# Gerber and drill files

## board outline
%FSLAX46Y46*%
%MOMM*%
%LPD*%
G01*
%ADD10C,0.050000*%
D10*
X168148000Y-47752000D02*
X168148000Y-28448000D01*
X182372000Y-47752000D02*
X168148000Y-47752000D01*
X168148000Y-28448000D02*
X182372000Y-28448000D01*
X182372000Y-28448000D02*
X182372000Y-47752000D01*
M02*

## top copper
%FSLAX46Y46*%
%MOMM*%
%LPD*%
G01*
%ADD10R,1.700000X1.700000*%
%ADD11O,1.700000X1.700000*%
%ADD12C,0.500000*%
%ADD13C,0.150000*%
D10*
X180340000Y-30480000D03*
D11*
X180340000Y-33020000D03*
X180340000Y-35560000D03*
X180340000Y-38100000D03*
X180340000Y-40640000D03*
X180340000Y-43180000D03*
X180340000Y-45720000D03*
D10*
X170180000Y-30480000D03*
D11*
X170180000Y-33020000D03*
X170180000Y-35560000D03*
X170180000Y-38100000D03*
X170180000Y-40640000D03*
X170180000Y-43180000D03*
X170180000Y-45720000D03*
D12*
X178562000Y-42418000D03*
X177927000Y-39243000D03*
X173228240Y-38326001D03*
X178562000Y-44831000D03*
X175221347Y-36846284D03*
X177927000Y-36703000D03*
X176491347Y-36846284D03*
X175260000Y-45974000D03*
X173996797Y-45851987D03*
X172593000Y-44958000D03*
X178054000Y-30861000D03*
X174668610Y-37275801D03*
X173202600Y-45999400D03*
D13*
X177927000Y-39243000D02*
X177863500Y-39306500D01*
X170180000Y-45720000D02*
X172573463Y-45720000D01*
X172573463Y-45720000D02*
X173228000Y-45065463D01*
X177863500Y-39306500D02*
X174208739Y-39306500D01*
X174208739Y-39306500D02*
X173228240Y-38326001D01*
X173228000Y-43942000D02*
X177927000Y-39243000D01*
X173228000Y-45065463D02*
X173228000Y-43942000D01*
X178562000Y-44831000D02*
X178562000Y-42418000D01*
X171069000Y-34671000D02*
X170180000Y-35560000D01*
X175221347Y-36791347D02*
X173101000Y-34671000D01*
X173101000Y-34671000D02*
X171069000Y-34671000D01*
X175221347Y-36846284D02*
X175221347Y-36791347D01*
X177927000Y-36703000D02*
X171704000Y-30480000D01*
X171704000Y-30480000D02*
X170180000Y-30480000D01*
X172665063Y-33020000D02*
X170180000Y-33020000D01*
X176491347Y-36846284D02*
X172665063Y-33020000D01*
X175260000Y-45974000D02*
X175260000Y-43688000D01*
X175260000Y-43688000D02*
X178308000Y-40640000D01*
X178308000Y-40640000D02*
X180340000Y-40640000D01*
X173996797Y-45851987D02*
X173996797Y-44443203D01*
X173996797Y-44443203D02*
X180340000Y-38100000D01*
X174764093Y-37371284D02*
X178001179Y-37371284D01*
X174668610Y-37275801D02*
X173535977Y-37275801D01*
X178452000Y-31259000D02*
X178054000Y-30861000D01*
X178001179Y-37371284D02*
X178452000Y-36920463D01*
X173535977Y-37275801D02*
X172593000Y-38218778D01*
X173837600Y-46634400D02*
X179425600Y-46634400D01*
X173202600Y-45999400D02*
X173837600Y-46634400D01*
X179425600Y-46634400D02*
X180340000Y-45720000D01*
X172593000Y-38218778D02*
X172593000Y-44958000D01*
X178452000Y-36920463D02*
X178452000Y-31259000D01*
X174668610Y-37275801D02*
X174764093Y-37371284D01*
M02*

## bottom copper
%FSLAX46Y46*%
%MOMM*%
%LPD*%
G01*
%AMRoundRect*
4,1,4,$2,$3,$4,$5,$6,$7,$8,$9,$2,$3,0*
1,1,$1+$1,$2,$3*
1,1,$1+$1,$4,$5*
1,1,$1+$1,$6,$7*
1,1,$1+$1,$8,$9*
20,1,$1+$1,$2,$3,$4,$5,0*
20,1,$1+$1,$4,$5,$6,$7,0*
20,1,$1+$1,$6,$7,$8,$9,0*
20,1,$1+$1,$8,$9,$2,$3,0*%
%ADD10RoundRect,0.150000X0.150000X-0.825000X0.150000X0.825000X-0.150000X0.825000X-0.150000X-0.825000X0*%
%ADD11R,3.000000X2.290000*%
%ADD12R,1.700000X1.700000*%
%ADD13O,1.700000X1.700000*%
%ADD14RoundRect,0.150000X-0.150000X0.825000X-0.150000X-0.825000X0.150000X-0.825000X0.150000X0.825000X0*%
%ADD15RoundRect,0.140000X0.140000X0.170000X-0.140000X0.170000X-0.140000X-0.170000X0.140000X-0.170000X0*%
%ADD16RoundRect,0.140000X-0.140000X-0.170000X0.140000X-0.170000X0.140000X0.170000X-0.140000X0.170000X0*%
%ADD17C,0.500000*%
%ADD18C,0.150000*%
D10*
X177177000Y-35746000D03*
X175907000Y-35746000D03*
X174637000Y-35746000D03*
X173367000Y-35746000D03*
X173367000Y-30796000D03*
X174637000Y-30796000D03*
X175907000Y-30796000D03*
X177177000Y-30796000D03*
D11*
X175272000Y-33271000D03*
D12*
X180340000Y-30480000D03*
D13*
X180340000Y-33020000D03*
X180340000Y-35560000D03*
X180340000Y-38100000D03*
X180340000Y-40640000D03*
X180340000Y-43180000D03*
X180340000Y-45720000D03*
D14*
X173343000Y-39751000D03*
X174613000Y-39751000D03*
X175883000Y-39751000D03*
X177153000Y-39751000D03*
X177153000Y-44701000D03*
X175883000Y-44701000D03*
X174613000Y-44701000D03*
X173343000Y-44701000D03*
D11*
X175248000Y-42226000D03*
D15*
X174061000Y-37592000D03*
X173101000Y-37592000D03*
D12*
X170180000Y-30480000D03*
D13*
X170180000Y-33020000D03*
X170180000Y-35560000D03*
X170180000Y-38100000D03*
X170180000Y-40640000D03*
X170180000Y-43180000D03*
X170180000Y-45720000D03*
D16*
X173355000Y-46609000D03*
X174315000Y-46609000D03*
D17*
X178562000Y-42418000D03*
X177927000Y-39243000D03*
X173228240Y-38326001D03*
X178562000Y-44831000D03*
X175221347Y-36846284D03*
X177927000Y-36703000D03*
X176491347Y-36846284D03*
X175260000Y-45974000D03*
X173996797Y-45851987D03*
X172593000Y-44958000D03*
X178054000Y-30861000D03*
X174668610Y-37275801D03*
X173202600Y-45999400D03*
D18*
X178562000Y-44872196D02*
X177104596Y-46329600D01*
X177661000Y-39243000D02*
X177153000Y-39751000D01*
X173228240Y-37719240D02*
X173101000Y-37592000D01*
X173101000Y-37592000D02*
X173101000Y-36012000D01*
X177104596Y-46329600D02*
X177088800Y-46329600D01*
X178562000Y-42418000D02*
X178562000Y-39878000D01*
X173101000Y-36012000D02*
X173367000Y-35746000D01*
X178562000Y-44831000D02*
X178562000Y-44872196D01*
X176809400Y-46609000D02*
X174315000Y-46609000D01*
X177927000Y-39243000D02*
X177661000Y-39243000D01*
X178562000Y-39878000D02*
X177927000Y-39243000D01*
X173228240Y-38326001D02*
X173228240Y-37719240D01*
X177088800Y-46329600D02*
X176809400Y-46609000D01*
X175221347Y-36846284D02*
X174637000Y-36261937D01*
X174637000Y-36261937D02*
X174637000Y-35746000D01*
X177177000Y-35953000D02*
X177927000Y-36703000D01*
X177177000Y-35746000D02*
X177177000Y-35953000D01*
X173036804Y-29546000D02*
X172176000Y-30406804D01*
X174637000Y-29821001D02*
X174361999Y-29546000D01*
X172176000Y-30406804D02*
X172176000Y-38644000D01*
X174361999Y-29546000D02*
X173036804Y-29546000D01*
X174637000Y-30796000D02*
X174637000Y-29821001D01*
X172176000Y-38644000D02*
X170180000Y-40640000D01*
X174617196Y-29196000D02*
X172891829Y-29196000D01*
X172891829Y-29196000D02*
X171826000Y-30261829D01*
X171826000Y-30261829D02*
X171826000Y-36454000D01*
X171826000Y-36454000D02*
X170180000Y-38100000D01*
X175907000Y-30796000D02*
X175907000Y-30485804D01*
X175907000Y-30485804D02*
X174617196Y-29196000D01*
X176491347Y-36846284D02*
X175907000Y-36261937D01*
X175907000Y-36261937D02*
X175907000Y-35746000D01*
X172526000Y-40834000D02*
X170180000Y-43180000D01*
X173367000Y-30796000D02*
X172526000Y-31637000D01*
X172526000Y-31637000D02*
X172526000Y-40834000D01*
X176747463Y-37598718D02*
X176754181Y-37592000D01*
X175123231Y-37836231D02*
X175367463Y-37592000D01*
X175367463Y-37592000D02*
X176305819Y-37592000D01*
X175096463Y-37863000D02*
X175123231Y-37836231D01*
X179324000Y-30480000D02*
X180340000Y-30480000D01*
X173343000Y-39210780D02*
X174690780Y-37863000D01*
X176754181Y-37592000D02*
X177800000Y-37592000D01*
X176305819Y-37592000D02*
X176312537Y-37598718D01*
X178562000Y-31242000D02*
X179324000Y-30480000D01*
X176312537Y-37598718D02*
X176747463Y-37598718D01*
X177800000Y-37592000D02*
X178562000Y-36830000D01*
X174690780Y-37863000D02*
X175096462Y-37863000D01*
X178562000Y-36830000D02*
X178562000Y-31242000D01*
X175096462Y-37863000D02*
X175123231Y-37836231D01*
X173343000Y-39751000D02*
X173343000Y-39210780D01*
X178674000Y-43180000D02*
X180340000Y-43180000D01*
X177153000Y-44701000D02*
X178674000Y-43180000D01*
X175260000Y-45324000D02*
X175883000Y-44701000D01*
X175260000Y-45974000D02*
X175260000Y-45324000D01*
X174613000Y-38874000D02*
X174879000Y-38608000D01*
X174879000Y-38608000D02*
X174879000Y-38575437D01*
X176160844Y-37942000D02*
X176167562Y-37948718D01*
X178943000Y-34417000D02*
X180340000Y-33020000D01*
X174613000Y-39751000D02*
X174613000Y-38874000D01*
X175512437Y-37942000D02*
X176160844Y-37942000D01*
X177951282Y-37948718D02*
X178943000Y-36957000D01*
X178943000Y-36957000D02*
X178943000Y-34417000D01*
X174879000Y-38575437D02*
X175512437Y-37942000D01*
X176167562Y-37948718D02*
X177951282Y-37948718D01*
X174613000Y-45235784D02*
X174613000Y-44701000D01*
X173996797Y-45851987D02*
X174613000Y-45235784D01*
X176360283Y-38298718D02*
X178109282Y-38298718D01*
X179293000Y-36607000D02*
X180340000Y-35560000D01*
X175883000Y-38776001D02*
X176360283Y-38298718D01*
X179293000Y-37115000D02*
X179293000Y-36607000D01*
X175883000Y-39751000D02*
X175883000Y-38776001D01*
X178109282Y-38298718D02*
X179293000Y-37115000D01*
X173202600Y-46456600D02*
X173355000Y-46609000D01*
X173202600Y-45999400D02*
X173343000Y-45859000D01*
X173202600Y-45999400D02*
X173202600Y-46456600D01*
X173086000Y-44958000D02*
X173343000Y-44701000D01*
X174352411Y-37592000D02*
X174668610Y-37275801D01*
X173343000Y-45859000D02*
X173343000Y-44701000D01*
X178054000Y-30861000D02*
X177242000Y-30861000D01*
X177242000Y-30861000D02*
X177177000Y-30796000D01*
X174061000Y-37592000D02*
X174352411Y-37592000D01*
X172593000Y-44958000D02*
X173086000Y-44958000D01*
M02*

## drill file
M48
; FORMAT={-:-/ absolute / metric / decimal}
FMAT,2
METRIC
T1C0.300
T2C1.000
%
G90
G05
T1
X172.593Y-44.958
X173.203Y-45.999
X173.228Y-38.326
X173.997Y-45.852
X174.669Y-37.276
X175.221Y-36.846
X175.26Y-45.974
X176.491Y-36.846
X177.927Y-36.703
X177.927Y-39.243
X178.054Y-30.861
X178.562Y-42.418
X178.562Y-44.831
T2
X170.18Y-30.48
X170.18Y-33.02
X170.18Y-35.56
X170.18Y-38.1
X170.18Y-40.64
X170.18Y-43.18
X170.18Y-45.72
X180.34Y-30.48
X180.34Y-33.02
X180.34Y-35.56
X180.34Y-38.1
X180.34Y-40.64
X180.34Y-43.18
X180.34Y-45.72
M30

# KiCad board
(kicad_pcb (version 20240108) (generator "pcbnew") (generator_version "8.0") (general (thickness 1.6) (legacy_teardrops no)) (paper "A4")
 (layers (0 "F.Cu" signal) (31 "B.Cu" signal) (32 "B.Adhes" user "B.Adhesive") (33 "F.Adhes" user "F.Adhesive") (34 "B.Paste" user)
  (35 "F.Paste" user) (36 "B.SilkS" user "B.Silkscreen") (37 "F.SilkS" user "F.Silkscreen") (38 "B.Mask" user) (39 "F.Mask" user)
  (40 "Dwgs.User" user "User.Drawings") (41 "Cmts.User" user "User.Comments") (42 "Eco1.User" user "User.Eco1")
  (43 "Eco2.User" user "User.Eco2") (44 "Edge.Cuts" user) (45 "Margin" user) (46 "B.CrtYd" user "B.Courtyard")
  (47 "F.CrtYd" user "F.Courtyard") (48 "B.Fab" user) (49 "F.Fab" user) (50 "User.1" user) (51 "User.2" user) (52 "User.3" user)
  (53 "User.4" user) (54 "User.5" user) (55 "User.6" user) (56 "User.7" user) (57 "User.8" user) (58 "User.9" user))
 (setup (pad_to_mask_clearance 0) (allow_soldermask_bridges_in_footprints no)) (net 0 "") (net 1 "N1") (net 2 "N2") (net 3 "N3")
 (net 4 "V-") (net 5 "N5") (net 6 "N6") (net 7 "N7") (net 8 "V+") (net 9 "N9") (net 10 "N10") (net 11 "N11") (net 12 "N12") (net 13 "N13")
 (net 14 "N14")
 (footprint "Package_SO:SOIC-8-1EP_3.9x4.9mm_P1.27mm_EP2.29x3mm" (layer "B.Cu") (at 175.272 33.271 90)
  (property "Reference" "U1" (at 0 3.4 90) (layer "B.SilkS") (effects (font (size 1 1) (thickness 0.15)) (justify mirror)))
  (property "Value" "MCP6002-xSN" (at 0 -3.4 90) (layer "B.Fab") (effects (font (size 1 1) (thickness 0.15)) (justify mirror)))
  (pad "" smd roundrect (at -0.57 -0.75 90) (size 0.92 1.21) (layers "B.Paste") (roundrect_rratio 0.25))
  (pad "" smd roundrect (at -0.57 0.75 90) (size 0.92 1.21) (layers "B.Paste") (roundrect_rratio 0.25))
  (pad "" smd roundrect (at 0.57 -0.75 90) (size 0.92 1.21) (layers "B.Paste") (roundrect_rratio 0.25))
  (pad "" smd roundrect (at 0.57 0.75 90) (size 0.92 1.21) (layers "B.Paste") (roundrect_rratio 0.25))
  (pad "1" smd roundrect (at -2.475 1.905 90) (size 1.95 0.6) (layers "B.Cu" "B.Paste" "B.Mask") (roundrect_rratio 0.25) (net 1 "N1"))
  (pad "2" smd roundrect (at -2.475 0.635 90) (size 1.95 0.6) (layers "B.Cu" "B.Paste" "B.Mask") (roundrect_rratio 0.25) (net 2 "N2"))
  (pad "3" smd roundrect (at -2.475 -0.635 90) (size 1.95 0.6) (layers "B.Cu" "B.Paste" "B.Mask") (roundrect_rratio 0.25) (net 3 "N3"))
  (pad "4" smd roundrect (at -2.475 -1.905 90) (size 1.95 0.6) (layers "B.Cu" "B.Paste" "B.Mask") (roundrect_rratio 0.25) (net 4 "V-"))
  (pad "5" smd roundrect (at 2.475 -1.905 90) (size 1.95 0.6) (layers "B.Cu" "B.Paste" "B.Mask") (roundrect_rratio 0.25) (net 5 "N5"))
  (pad "6" smd roundrect (at 2.475 -0.635 90) (size 1.95 0.6) (layers "B.Cu" "B.Paste" "B.Mask") (roundrect_rratio 0.25) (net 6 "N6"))
  (pad "7" smd roundrect (at 2.475 0.635 90) (size 1.95 0.6) (layers "B.Cu" "B.Paste" "B.Mask") (roundrect_rratio 0.25) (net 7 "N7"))
  (pad "8" smd roundrect (at 2.475 1.905 90) (size 1.95 0.6) (layers "B.Cu" "B.Paste" "B.Mask") (roundrect_rratio 0.25) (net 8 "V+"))
  (pad "9" smd rect (at 0 0 90) (size 2.29 3) (layers "B.Cu" "B.Mask") (zone_connect 2)))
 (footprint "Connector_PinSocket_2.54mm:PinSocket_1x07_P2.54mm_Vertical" (layer "B.Cu") (at 180.34 30.48 180)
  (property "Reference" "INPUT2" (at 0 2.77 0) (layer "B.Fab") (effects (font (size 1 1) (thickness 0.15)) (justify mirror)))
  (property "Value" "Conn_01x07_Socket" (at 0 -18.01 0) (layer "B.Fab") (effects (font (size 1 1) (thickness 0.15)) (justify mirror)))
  (pad "1" thru_hole rect (at 0 0 180) (size 1.7 1.7) (drill 1) (layers "*.Cu" "*.Mask") (remove_unused_layers no) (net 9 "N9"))
  (pad "2" thru_hole oval (at 0 -2.54 180) (size 1.7 1.7) (drill 1) (layers "*.Cu" "*.Mask") (remove_unused_layers no) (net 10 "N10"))
  (pad "3" thru_hole oval (at 0 -5.08 180) (size 1.7 1.7) (drill 1) (layers "*.Cu" "*.Mask") (remove_unused_layers no) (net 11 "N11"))
  (pad "4" thru_hole oval (at 0 -7.62 180) (size 1.7 1.7) (drill 1) (layers "*.Cu" "*.Mask") (remove_unused_layers no) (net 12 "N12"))
  (pad "5" thru_hole oval (at 0 -10.16 180) (size 1.7 1.7) (drill 1) (layers "*.Cu" "*.Mask") (remove_unused_layers no) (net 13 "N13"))
  (pad "6" thru_hole oval (at 0 -12.7 180) (size 1.7 1.7) (drill 1) (layers "*.Cu" "*.Mask") (remove_unused_layers no) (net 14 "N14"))
  (pad "7" thru_hole oval (at 0 -15.24 180) (size 1.7 1.7) (drill 1) (layers "*.Cu" "*.Mask") (remove_unused_layers no) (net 8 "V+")))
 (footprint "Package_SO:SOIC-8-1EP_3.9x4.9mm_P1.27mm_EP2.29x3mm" (layer "B.Cu") (at 175.248 42.226 -90)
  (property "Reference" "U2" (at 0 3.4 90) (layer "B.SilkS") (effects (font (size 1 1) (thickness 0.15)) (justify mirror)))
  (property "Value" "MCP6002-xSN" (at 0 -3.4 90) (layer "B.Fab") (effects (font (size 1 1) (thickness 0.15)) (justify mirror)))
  (pad "" smd roundrect (at -0.57 -0.75 270) (size 0.92 1.21) (layers "B.Paste") (roundrect_rratio 0.25))
  (pad "" smd roundrect (at -0.57 0.75 270) (size 0.92 1.21) (layers "B.Paste") (roundrect_rratio 0.25))
  (pad "" smd roundrect (at 0.57 -0.75 270) (size 0.92 1.21) (layers "B.Paste") (roundrect_rratio 0.25))
  (pad "" smd roundrect (at 0.57 0.75 270) (size 0.92 1.21) (layers "B.Paste") (roundrect_rratio 0.25))
  (pad "1" smd roundrect (at -2.475 1.905 270) (size 1.95 0.6) (layers "B.Cu" "B.Paste" "B.Mask") (roundrect_rratio 0.25) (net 9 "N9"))
  (pad "2" smd roundrect (at -2.475 0.635 270) (size 1.95 0.6) (layers "B.Cu" "B.Paste" "B.Mask") (roundrect_rratio 0.25) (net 10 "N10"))
  (pad "3" smd roundrect (at -2.475 -0.635 270) (size 1.95 0.6) (layers "B.Cu" "B.Paste" "B.Mask") (roundrect_rratio 0.25) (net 11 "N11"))
  (pad "4" smd roundrect (at -2.475 -1.905 270) (size 1.95 0.6) (layers "B.Cu" "B.Paste" "B.Mask") (roundrect_rratio 0.25) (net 4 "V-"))
  (pad "5" smd roundrect (at 2.475 -1.905 270) (size 1.95 0.6) (layers "B.Cu" "B.Paste" "B.Mask") (roundrect_rratio 0.25) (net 14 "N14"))
  (pad "6" smd roundrect (at 2.475 -0.635 270) (size 1.95 0.6) (layers "B.Cu" "B.Paste" "B.Mask") (roundrect_rratio 0.25) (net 13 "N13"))
  (pad "7" smd roundrect (at 2.475 0.635 270) (size 1.95 0.6) (layers "B.Cu" "B.Paste" "B.Mask") (roundrect_rratio 0.25) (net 12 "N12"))
  (pad "8" smd roundrect (at 2.475 1.905 270) (size 1.95 0.6) (layers "B.Cu" "B.Paste" "B.Mask") (roundrect_rratio 0.25) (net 8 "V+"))
  (pad "9" smd rect (at 0 0 270) (size 2.29 3) (layers "B.Cu" "B.Mask") (zone_connect 2)))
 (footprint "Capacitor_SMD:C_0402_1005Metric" (layer "B.Cu") (at 173.581 37.592 180)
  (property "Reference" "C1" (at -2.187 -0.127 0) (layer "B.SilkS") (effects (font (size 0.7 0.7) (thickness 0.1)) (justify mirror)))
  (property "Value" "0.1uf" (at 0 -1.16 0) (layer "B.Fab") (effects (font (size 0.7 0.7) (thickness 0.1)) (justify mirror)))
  (pad "1" smd roundrect (at -0.48 0 180) (size 0.56 0.62) (layers "B.Cu" "B.Paste" "B.Mask") (roundrect_rratio 0.25) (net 8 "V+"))
  (pad "2" smd roundrect (at 0.48 0 180) (size 0.56 0.62) (layers "B.Cu" "B.Paste" "B.Mask") (roundrect_rratio 0.25) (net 4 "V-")))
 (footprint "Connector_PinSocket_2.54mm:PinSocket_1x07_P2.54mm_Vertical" (layer "B.Cu") (at 170.18 30.48 180)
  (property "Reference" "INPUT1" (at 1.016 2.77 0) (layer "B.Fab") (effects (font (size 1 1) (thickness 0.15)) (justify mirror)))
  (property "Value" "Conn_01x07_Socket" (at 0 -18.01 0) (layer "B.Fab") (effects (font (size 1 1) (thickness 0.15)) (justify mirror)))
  (pad "1" thru_hole rect (at 0 0 180) (size 1.7 1.7) (drill 1) (layers "*.Cu" "*.Mask") (remove_unused_layers no) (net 1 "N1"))
  (pad "2" thru_hole oval (at 0 -2.54 180) (size 1.7 1.7) (drill 1) (layers "*.Cu" "*.Mask") (remove_unused_layers no) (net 2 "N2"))
  (pad "3" thru_hole oval (at 0 -5.08 180) (size 1.7 1.7) (drill 1) (layers "*.Cu" "*.Mask") (remove_unused_layers no) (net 3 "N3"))
  (pad "4" thru_hole oval (at 0 -7.62 180) (size 1.7 1.7) (drill 1) (layers "*.Cu" "*.Mask") (remove_unused_layers no) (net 7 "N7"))
  (pad "5" thru_hole oval (at 0 -10.16 180) (size 1.7 1.7) (drill 1) (layers "*.Cu" "*.Mask") (remove_unused_layers no) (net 6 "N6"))
  (pad "6" thru_hole oval (at 0 -12.7 180) (size 1.7 1.7) (drill 1) (layers "*.Cu" "*.Mask") (remove_unused_layers no) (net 5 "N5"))
  (pad "7" thru_hole oval (at 0 -15.24 180) (size 1.7 1.7) (drill 1) (layers "*.Cu" "*.Mask") (remove_unused_layers no) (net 4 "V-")))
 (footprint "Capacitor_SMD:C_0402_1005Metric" (layer "B.Cu") (at 173.835 46.609)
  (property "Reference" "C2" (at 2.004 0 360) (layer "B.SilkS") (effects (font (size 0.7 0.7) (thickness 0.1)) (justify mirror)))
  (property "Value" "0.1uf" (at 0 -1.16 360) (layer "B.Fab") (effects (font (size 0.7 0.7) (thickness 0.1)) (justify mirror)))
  (pad "1" smd roundrect (at -0.48 0) (size 0.56 0.62) (layers "B.Cu" "B.Paste" "B.Mask") (roundrect_rratio 0.25) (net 8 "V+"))
  (pad "2" smd roundrect (at 0.48 0) (size 0.56 0.62) (layers "B.Cu" "B.Paste" "B.Mask") (roundrect_rratio 0.25) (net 4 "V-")))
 (gr_line (start 168.148 47.752) (end 168.148 28.448) (stroke (width 0.05) (type default)) (layer "Edge.Cuts"))
 (gr_line (start 182.372 47.752) (end 168.148 47.752) (stroke (width 0.05) (type default)) (layer "Edge.Cuts"))
 (gr_line (start 168.148 28.448) (end 182.372 28.448) (stroke (width 0.05) (type default)) (layer "Edge.Cuts"))
 (gr_line (start 182.372 28.448) (end 182.372 47.752) (stroke (width 0.05) (type default)) (layer "Edge.Cuts"))
 (segment (start 177.927 39.243) (end 177.8635 39.3065) (width 0.15) (layer "F.Cu") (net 4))
 (segment (start 170.18 45.72) (end 172.573463 45.72) (width 0.15) (layer "F.Cu") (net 4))
 (segment (start 172.573463 45.72) (end 173.228 45.065463) (width 0.15) (layer "F.Cu") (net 4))
 (segment (start 177.8635 39.3065) (end 174.208739 39.3065) (width 0.15) (layer "F.Cu") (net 4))
 (segment (start 174.208739 39.3065) (end 173.22824 38.326001) (width 0.15) (layer "F.Cu") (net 4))
 (segment (start 173.228 43.942) (end 177.927 39.243) (width 0.15) (layer "F.Cu") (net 4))
 (segment (start 173.228 45.065463) (end 173.228 43.942) (width 0.15) (layer "F.Cu") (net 4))
 (segment (start 178.562 44.831) (end 178.562 42.418) (width 0.15) (layer "F.Cu") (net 4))
 (via (at 178.562 42.418) (size 0.5) (drill 0.3) (layers "F.Cu" "B.Cu") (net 4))
 (via (at 177.927 39.243) (size 0.5) (drill 0.3) (layers "F.Cu" "B.Cu") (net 4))
 (via (at 173.22824 38.326001) (size 0.5) (drill 0.3) (layers "F.Cu" "B.Cu") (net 4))
 (via (at 178.562 44.831) (size 0.5) (drill 0.3) (layers "F.Cu" "B.Cu") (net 4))
 (segment (start 178.562 44.872196) (end 177.104596 46.3296) (width 0.15) (layer "B.Cu") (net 4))
 (segment (start 177.661 39.243) (end 177.153 39.751) (width 0.15) (layer "B.Cu") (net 4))
 (segment (start 173.22824 37.71924) (end 173.101 37.592) (width 0.15) (layer "B.Cu") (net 4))
 (segment (start 173.101 37.592) (end 173.101 36.012) (width 0.15) (layer "B.Cu") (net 4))
 (segment (start 177.104596 46.3296) (end 177.0888 46.3296) (width 0.15) (layer "B.Cu") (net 4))
 (segment (start 178.562 42.418) (end 178.562 39.878) (width 0.15) (layer "B.Cu") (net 4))
 (segment (start 173.101 36.012) (end 173.367 35.746) (width 0.15) (layer "B.Cu") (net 4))
 (segment (start 178.562 44.831) (end 178.562 44.872196) (width 0.15) (layer "B.Cu") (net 4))
 (segment (start 176.8094 46.609) (end 174.315 46.609) (width 0.15) (layer "B.Cu") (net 4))
 (segment (start 177.927 39.243) (end 177.661 39.243) (width 0.15) (layer "B.Cu") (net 4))
 (segment (start 178.562 39.878) (end 177.927 39.243) (width 0.15) (layer "B.Cu") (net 4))
 (segment (start 173.22824 38.326001) (end 173.22824 37.71924) (width 0.15) (layer "B.Cu") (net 4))
 (segment (start 177.0888 46.3296) (end 176.8094 46.609) (width 0.15) (layer "B.Cu") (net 4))
 (segment (start 171.069 34.671) (end 170.18 35.56) (width 0.15) (layer "F.Cu") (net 3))
 (segment (start 175.221347 36.791347) (end 173.101 34.671) (width 0.15) (layer "F.Cu") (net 3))
 (segment (start 173.101 34.671) (end 171.069 34.671) (width 0.15) (layer "F.Cu") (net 3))
 (segment (start 175.221347 36.846284) (end 175.221347 36.791347) (width 0.15) (layer "F.Cu") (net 3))
 (via (at 175.221347 36.846284) (size 0.5) (drill 0.3) (layers "F.Cu" "B.Cu") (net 3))
 (segment (start 175.221347 36.846284) (end 174.637 36.261937) (width 0.15) (layer "B.Cu") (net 3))
 (segment (start 174.637 36.261937) (end 174.637 35.746) (width 0.15) (layer "B.Cu") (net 3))
 (segment (start 177.927 36.703) (end 171.704 30.48) (width 0.15) (layer "F.Cu") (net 1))
 (segment (start 171.704 30.48) (end 170.18 30.48) (width 0.15) (layer "F.Cu") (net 1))
 (via (at 177.927 36.703) (size 0.5) (drill 0.3) (layers "F.Cu" "B.Cu") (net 1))
 (segment (start 177.177 35.953) (end 177.927 36.703) (width 0.15) (layer "B.Cu") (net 1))
 (segment (start 177.177 35.746) (end 177.177 35.953) (width 0.15) (layer "B.Cu") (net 1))
 (segment (start 173.036804 29.546) (end 172.176 30.406804) (width 0.15) (layer "B.Cu") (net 6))
 (segment (start 174.637 29.821001) (end 174.361999 29.546) (width 0.15) (layer "B.Cu") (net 6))
 (segment (start 172.176 30.406804) (end 172.176 38.644) (width 0.15) (layer "B.Cu") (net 6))
 (segment (start 174.361999 29.546) (end 173.036804 29.546) (width 0.15) (layer "B.Cu") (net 6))
 (segment (start 174.637 30.796) (end 174.637 29.821001) (width 0.15) (layer "B.Cu") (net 6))
 (segment (start 172.176 38.644) (end 170.18 40.64) (width 0.15) (layer "B.Cu") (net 6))
 (segment (start 174.617196 29.196) (end 172.891829 29.196) (width 0.15) (layer "B.Cu") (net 7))
 (segment (start 172.891829 29.196) (end 171.826 30.261829) (width 0.15) (layer "B.Cu") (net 7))
 (segment (start 171.826 30.261829) (end 171.826 36.454) (width 0.15) (layer "B.Cu") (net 7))
 (segment (start 171.826 36.454) (end 170.18 38.1) (width 0.15) (layer "B.Cu") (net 7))
 (segment (start 175.907 30.796) (end 175.907 30.485804) (width 0.15) (layer "B.Cu") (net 7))
 (segment (start 175.907 30.485804) (end 174.617196 29.196) (width 0.15) (layer "B.Cu") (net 7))
 (segment (start 172.665063 33.02) (end 170.18 33.02) (width 0.15) (layer "F.Cu") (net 2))
 (segment (start 176.491347 36.846284) (end 172.665063 33.02) (width 0.15) (layer "F.Cu") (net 2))
 (via (at 176.491347 36.846284) (size 0.5) (drill 0.3) (layers "F.Cu" "B.Cu") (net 2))
 (segment (start 176.491347 36.846284) (end 175.907 36.261937) (width 0.15) (layer "B.Cu") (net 2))
 (segment (start 175.907 36.261937) (end 175.907 35.746) (width 0.15) (layer "B.Cu") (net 2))
 (segment (start 172.526 40.834) (end 170.18 43.18) (width 0.15) (layer "B.Cu") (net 5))
 (segment (start 173.367 30.796) (end 172.526 31.637) (width 0.15) (layer "B.Cu") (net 5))
 (segment (start 172.526 31.637) (end 172.526 40.834) (width 0.15) (layer "B.Cu") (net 5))
 (segment (start 176.747463 37.598718) (end 176.754181 37.592) (width 0.15) (layer "B.Cu") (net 9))
 (segment (start 175.123231 37.836231) (end 175.367463 37.592) (width 0.15) (layer "B.Cu") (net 9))
 (segment (start 175.367463 37.592) (end 176.305819 37.592) (width 0.15) (layer "B.Cu") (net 9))
 (segment (start 175.096463 37.863) (end 175.123231 37.836231) (width 0.15) (layer "B.Cu") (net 9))
 (segment (start 179.324 30.48) (end 180.34 30.48) (width 0.15) (layer "B.Cu") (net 9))
 (segment (start 173.343 39.21078) (end 174.69078 37.863) (width 0.15) (layer "B.Cu") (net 9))
 (segment (start 176.754181 37.592) (end 177.8 37.592) (width 0.15) (layer "B.Cu") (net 9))
 (segment (start 176.305819 37.592) (end 176.312537 37.598718) (width 0.15) (layer "B.Cu") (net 9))
 (segment (start 178.562 31.242) (end 179.324 30.48) (width 0.15) (layer "B.Cu") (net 9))
 (segment (start 176.312537 37.598718) (end 176.747463 37.598718) (width 0.15) (layer "B.Cu") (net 9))
 (segment (start 177.8 37.592) (end 178.562 36.83) (width 0.15) (layer "B.Cu") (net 9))
 (segment (start 174.69078 37.863) (end 175.096462 37.863) (width 0.15) (layer "B.Cu") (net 9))
 (segment (start 178.562 36.83) (end 178.562 31.242) (width 0.15) (layer "B.Cu") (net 9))
 (segment (start 175.096462 37.863) (end 175.123231 37.836231) (width 0.15) (layer "B.Cu") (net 9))
 (segment (start 173.343 39.751) (end 173.343 39.21078) (width 0.15) (layer "B.Cu") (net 9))
 (segment (start 178.674 43.18) (end 180.34 43.18) (width 0.15) (layer "B.Cu") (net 14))
 (segment (start 177.153 44.701) (end 178.674 43.18) (width 0.15) (layer "B.Cu") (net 14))
 (segment (start 175.26 45.974) (end 175.26 43.688) (width 0.15) (layer "F.Cu") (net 13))
 (segment (start 175.26 43.688) (end 178.308 40.64) (width 0.15) (layer "F.Cu") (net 13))
 (segment (start 178.308 40.64) (end 180.34 40.64) (width 0.15) (layer "F.Cu") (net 13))
 (via (at 175.26 45.974) (size 0.5) (drill 0.3) (layers "F.Cu" "B.Cu") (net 13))
 (segment (start 175.26 45.324) (end 175.883 44.701) (width 0.15) (layer "B.Cu") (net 13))
 (segment (start 175.26 45.974) (end 175.26 45.324) (width 0.15) (layer "B.Cu") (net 13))
 (segment (start 174.613 38.874) (end 174.879 38.608) (width 0.15) (layer "B.Cu") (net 10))
 (segment (start 174.879 38.608) (end 174.879 38.575437) (width 0.15) (layer "B.Cu") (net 10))
 (segment (start 176.160844 37.942) (end 176.167562 37.948718) (width 0.15) (layer "B.Cu") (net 10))
 (segment (start 178.943 34.417) (end 180.34 33.02) (width 0.15) (layer "B.Cu") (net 10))
 (segment (start 174.613 39.751) (end 174.613 38.874) (width 0.15) (layer "B.Cu") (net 10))
 (segment (start 175.512437 37.942) (end 176.160844 37.942) (width 0.15) (layer "B.Cu") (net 10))
 (segment (start 177.951282 37.948718) (end 178.943 36.957) (width 0.15) (layer "B.Cu") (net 10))
 (segment (start 178.943 36.957) (end 178.943 34.417) (width 0.15) (layer "B.Cu") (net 10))
 (segment (start 174.879 38.575437) (end 175.512437 37.942) (width 0.15) (layer "B.Cu") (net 10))
 (segment (start 176.167562 37.948718) (end 177.951282 37.948718) (width 0.15) (layer "B.Cu") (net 10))
 (segment (start 173.996797 45.851987) (end 173.996797 44.443203) (width 0.15) (layer "F.Cu") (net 12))
 (segment (start 173.996797 44.443203) (end 180.34 38.1) (width 0.15) (layer "F.Cu") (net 12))
 (via (at 173.996797 45.851987) (size 0.5) (drill 0.3) (layers "F.Cu" "B.Cu") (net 12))
 (segment (start 174.613 45.235784) (end 174.613 44.701) (width 0.15) (layer "B.Cu") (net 12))
 (segment (start 173.996797 45.851987) (end 174.613 45.235784) (width 0.15) (layer "B.Cu") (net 12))
 (segment (start 176.360283 38.298718) (end 178.109282 38.298718) (width 0.15) (layer "B.Cu") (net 11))
 (segment (start 179.293 36.607) (end 180.34 35.56) (width 0.15) (layer "B.Cu") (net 11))
 (segment (start 175.883 38.776001) (end 176.360283 38.298718) (width 0.15) (layer "B.Cu") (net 11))
 (segment (start 179.293 37.115) (end 179.293 36.607) (width 0.15) (layer "B.Cu") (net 11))
 (segment (start 175.883 39.751) (end 175.883 38.776001) (width 0.15) (layer "B.Cu") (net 11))
 (segment (start 178.109282 38.298718) (end 179.293 37.115) (width 0.15) (layer "B.Cu") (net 11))
 (segment (start 174.764093 37.371284) (end 178.001179 37.371284) (width 0.15) (layer "F.Cu") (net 8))
 (segment (start 174.66861 37.275801) (end 173.535977 37.275801) (width 0.15) (layer "F.Cu") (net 8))
 (segment (start 178.452 31.259) (end 178.054 30.861) (width 0.15) (layer "F.Cu") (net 8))
 (segment (start 178.001179 37.371284) (end 178.452 36.920463) (width 0.15) (layer "F.Cu") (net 8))
 (segment (start 173.535977 37.275801) (end 172.593 38.218778) (width 0.15) (layer "F.Cu") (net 8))
 (segment (start 173.8376 46.6344) (end 179.4256 46.6344) (width 0.15) (layer "F.Cu") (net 8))
 (segment (start 173.2026 45.9994) (end 173.8376 46.6344) (width 0.15) (layer "F.Cu") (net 8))
 (segment (start 179.4256 46.6344) (end 180.34 45.72) (width 0.15) (layer "F.Cu") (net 8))
 (segment (start 172.593 38.218778) (end 172.593 44.958) (width 0.15) (layer "F.Cu") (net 8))
 (segment (start 178.452 36.920463) (end 178.452 31.259) (width 0.15) (layer "F.Cu") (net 8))
 (segment (start 174.66861 37.275801) (end 174.764093 37.371284) (width 0.15) (layer "F.Cu") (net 8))
 (via (at 172.593 44.958) (size 0.5) (drill 0.3) (layers "F.Cu" "B.Cu") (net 8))
 (via (at 178.054 30.861) (size 0.5) (drill 0.3) (layers "F.Cu" "B.Cu") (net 8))
 (via (at 174.66861 37.275801) (size 0.5) (drill 0.3) (layers "F.Cu" "B.Cu") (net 8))
 (via (at 173.2026 45.9994) (size 0.5) (drill 0.3) (layers "F.Cu" "B.Cu") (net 8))
 (segment (start 173.2026 46.4566) (end 173.355 46.609) (width 0.15) (layer "B.Cu") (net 8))
 (segment (start 173.2026 45.9994) (end 173.343 45.859) (width 0.15) (layer "B.Cu") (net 8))
 (segment (start 173.2026 45.9994) (end 173.2026 46.4566) (width 0.15) (layer "B.Cu") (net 8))
 (segment (start 173.086 44.958) (end 173.343 44.701) (width 0.15) (layer "B.Cu") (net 8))
 (segment (start 174.352411 37.592) (end 174.66861 37.275801) (width 0.15) (layer "B.Cu") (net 8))
 (segment (start 173.343 45.859) (end 173.343 44.701) (width 0.15) (layer "B.Cu") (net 8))
 (segment (start 178.054 30.861) (end 177.242 30.861) (width 0.15) (layer "B.Cu") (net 8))
 (segment (start 177.242 30.861) (end 177.177 30.796) (width 0.15) (layer "B.Cu") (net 8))
 (segment (start 174.061 37.592) (end 174.352411 37.592) (width 0.15) (layer "B.Cu") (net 8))
 (segment (start 172.593 44.958) (end 173.086 44.958) (width 0.15) (layer "B.Cu") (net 8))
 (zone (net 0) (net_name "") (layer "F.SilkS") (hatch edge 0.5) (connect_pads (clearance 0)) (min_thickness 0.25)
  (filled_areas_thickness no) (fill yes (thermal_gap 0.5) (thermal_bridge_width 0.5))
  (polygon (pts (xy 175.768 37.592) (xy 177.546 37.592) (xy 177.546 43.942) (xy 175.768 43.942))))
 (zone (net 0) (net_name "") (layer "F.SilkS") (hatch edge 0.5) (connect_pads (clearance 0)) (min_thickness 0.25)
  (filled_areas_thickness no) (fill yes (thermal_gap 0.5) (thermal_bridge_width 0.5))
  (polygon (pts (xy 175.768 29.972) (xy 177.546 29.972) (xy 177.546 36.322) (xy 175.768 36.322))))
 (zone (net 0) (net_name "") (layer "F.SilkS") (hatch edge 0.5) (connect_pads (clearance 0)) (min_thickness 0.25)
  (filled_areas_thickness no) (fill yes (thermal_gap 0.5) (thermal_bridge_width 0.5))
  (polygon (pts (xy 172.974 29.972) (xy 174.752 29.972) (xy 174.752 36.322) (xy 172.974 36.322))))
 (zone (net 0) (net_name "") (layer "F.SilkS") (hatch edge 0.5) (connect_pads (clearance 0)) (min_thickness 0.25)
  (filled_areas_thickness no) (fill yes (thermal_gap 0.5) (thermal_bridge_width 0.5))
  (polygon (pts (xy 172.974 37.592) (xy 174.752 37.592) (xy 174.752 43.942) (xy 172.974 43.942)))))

